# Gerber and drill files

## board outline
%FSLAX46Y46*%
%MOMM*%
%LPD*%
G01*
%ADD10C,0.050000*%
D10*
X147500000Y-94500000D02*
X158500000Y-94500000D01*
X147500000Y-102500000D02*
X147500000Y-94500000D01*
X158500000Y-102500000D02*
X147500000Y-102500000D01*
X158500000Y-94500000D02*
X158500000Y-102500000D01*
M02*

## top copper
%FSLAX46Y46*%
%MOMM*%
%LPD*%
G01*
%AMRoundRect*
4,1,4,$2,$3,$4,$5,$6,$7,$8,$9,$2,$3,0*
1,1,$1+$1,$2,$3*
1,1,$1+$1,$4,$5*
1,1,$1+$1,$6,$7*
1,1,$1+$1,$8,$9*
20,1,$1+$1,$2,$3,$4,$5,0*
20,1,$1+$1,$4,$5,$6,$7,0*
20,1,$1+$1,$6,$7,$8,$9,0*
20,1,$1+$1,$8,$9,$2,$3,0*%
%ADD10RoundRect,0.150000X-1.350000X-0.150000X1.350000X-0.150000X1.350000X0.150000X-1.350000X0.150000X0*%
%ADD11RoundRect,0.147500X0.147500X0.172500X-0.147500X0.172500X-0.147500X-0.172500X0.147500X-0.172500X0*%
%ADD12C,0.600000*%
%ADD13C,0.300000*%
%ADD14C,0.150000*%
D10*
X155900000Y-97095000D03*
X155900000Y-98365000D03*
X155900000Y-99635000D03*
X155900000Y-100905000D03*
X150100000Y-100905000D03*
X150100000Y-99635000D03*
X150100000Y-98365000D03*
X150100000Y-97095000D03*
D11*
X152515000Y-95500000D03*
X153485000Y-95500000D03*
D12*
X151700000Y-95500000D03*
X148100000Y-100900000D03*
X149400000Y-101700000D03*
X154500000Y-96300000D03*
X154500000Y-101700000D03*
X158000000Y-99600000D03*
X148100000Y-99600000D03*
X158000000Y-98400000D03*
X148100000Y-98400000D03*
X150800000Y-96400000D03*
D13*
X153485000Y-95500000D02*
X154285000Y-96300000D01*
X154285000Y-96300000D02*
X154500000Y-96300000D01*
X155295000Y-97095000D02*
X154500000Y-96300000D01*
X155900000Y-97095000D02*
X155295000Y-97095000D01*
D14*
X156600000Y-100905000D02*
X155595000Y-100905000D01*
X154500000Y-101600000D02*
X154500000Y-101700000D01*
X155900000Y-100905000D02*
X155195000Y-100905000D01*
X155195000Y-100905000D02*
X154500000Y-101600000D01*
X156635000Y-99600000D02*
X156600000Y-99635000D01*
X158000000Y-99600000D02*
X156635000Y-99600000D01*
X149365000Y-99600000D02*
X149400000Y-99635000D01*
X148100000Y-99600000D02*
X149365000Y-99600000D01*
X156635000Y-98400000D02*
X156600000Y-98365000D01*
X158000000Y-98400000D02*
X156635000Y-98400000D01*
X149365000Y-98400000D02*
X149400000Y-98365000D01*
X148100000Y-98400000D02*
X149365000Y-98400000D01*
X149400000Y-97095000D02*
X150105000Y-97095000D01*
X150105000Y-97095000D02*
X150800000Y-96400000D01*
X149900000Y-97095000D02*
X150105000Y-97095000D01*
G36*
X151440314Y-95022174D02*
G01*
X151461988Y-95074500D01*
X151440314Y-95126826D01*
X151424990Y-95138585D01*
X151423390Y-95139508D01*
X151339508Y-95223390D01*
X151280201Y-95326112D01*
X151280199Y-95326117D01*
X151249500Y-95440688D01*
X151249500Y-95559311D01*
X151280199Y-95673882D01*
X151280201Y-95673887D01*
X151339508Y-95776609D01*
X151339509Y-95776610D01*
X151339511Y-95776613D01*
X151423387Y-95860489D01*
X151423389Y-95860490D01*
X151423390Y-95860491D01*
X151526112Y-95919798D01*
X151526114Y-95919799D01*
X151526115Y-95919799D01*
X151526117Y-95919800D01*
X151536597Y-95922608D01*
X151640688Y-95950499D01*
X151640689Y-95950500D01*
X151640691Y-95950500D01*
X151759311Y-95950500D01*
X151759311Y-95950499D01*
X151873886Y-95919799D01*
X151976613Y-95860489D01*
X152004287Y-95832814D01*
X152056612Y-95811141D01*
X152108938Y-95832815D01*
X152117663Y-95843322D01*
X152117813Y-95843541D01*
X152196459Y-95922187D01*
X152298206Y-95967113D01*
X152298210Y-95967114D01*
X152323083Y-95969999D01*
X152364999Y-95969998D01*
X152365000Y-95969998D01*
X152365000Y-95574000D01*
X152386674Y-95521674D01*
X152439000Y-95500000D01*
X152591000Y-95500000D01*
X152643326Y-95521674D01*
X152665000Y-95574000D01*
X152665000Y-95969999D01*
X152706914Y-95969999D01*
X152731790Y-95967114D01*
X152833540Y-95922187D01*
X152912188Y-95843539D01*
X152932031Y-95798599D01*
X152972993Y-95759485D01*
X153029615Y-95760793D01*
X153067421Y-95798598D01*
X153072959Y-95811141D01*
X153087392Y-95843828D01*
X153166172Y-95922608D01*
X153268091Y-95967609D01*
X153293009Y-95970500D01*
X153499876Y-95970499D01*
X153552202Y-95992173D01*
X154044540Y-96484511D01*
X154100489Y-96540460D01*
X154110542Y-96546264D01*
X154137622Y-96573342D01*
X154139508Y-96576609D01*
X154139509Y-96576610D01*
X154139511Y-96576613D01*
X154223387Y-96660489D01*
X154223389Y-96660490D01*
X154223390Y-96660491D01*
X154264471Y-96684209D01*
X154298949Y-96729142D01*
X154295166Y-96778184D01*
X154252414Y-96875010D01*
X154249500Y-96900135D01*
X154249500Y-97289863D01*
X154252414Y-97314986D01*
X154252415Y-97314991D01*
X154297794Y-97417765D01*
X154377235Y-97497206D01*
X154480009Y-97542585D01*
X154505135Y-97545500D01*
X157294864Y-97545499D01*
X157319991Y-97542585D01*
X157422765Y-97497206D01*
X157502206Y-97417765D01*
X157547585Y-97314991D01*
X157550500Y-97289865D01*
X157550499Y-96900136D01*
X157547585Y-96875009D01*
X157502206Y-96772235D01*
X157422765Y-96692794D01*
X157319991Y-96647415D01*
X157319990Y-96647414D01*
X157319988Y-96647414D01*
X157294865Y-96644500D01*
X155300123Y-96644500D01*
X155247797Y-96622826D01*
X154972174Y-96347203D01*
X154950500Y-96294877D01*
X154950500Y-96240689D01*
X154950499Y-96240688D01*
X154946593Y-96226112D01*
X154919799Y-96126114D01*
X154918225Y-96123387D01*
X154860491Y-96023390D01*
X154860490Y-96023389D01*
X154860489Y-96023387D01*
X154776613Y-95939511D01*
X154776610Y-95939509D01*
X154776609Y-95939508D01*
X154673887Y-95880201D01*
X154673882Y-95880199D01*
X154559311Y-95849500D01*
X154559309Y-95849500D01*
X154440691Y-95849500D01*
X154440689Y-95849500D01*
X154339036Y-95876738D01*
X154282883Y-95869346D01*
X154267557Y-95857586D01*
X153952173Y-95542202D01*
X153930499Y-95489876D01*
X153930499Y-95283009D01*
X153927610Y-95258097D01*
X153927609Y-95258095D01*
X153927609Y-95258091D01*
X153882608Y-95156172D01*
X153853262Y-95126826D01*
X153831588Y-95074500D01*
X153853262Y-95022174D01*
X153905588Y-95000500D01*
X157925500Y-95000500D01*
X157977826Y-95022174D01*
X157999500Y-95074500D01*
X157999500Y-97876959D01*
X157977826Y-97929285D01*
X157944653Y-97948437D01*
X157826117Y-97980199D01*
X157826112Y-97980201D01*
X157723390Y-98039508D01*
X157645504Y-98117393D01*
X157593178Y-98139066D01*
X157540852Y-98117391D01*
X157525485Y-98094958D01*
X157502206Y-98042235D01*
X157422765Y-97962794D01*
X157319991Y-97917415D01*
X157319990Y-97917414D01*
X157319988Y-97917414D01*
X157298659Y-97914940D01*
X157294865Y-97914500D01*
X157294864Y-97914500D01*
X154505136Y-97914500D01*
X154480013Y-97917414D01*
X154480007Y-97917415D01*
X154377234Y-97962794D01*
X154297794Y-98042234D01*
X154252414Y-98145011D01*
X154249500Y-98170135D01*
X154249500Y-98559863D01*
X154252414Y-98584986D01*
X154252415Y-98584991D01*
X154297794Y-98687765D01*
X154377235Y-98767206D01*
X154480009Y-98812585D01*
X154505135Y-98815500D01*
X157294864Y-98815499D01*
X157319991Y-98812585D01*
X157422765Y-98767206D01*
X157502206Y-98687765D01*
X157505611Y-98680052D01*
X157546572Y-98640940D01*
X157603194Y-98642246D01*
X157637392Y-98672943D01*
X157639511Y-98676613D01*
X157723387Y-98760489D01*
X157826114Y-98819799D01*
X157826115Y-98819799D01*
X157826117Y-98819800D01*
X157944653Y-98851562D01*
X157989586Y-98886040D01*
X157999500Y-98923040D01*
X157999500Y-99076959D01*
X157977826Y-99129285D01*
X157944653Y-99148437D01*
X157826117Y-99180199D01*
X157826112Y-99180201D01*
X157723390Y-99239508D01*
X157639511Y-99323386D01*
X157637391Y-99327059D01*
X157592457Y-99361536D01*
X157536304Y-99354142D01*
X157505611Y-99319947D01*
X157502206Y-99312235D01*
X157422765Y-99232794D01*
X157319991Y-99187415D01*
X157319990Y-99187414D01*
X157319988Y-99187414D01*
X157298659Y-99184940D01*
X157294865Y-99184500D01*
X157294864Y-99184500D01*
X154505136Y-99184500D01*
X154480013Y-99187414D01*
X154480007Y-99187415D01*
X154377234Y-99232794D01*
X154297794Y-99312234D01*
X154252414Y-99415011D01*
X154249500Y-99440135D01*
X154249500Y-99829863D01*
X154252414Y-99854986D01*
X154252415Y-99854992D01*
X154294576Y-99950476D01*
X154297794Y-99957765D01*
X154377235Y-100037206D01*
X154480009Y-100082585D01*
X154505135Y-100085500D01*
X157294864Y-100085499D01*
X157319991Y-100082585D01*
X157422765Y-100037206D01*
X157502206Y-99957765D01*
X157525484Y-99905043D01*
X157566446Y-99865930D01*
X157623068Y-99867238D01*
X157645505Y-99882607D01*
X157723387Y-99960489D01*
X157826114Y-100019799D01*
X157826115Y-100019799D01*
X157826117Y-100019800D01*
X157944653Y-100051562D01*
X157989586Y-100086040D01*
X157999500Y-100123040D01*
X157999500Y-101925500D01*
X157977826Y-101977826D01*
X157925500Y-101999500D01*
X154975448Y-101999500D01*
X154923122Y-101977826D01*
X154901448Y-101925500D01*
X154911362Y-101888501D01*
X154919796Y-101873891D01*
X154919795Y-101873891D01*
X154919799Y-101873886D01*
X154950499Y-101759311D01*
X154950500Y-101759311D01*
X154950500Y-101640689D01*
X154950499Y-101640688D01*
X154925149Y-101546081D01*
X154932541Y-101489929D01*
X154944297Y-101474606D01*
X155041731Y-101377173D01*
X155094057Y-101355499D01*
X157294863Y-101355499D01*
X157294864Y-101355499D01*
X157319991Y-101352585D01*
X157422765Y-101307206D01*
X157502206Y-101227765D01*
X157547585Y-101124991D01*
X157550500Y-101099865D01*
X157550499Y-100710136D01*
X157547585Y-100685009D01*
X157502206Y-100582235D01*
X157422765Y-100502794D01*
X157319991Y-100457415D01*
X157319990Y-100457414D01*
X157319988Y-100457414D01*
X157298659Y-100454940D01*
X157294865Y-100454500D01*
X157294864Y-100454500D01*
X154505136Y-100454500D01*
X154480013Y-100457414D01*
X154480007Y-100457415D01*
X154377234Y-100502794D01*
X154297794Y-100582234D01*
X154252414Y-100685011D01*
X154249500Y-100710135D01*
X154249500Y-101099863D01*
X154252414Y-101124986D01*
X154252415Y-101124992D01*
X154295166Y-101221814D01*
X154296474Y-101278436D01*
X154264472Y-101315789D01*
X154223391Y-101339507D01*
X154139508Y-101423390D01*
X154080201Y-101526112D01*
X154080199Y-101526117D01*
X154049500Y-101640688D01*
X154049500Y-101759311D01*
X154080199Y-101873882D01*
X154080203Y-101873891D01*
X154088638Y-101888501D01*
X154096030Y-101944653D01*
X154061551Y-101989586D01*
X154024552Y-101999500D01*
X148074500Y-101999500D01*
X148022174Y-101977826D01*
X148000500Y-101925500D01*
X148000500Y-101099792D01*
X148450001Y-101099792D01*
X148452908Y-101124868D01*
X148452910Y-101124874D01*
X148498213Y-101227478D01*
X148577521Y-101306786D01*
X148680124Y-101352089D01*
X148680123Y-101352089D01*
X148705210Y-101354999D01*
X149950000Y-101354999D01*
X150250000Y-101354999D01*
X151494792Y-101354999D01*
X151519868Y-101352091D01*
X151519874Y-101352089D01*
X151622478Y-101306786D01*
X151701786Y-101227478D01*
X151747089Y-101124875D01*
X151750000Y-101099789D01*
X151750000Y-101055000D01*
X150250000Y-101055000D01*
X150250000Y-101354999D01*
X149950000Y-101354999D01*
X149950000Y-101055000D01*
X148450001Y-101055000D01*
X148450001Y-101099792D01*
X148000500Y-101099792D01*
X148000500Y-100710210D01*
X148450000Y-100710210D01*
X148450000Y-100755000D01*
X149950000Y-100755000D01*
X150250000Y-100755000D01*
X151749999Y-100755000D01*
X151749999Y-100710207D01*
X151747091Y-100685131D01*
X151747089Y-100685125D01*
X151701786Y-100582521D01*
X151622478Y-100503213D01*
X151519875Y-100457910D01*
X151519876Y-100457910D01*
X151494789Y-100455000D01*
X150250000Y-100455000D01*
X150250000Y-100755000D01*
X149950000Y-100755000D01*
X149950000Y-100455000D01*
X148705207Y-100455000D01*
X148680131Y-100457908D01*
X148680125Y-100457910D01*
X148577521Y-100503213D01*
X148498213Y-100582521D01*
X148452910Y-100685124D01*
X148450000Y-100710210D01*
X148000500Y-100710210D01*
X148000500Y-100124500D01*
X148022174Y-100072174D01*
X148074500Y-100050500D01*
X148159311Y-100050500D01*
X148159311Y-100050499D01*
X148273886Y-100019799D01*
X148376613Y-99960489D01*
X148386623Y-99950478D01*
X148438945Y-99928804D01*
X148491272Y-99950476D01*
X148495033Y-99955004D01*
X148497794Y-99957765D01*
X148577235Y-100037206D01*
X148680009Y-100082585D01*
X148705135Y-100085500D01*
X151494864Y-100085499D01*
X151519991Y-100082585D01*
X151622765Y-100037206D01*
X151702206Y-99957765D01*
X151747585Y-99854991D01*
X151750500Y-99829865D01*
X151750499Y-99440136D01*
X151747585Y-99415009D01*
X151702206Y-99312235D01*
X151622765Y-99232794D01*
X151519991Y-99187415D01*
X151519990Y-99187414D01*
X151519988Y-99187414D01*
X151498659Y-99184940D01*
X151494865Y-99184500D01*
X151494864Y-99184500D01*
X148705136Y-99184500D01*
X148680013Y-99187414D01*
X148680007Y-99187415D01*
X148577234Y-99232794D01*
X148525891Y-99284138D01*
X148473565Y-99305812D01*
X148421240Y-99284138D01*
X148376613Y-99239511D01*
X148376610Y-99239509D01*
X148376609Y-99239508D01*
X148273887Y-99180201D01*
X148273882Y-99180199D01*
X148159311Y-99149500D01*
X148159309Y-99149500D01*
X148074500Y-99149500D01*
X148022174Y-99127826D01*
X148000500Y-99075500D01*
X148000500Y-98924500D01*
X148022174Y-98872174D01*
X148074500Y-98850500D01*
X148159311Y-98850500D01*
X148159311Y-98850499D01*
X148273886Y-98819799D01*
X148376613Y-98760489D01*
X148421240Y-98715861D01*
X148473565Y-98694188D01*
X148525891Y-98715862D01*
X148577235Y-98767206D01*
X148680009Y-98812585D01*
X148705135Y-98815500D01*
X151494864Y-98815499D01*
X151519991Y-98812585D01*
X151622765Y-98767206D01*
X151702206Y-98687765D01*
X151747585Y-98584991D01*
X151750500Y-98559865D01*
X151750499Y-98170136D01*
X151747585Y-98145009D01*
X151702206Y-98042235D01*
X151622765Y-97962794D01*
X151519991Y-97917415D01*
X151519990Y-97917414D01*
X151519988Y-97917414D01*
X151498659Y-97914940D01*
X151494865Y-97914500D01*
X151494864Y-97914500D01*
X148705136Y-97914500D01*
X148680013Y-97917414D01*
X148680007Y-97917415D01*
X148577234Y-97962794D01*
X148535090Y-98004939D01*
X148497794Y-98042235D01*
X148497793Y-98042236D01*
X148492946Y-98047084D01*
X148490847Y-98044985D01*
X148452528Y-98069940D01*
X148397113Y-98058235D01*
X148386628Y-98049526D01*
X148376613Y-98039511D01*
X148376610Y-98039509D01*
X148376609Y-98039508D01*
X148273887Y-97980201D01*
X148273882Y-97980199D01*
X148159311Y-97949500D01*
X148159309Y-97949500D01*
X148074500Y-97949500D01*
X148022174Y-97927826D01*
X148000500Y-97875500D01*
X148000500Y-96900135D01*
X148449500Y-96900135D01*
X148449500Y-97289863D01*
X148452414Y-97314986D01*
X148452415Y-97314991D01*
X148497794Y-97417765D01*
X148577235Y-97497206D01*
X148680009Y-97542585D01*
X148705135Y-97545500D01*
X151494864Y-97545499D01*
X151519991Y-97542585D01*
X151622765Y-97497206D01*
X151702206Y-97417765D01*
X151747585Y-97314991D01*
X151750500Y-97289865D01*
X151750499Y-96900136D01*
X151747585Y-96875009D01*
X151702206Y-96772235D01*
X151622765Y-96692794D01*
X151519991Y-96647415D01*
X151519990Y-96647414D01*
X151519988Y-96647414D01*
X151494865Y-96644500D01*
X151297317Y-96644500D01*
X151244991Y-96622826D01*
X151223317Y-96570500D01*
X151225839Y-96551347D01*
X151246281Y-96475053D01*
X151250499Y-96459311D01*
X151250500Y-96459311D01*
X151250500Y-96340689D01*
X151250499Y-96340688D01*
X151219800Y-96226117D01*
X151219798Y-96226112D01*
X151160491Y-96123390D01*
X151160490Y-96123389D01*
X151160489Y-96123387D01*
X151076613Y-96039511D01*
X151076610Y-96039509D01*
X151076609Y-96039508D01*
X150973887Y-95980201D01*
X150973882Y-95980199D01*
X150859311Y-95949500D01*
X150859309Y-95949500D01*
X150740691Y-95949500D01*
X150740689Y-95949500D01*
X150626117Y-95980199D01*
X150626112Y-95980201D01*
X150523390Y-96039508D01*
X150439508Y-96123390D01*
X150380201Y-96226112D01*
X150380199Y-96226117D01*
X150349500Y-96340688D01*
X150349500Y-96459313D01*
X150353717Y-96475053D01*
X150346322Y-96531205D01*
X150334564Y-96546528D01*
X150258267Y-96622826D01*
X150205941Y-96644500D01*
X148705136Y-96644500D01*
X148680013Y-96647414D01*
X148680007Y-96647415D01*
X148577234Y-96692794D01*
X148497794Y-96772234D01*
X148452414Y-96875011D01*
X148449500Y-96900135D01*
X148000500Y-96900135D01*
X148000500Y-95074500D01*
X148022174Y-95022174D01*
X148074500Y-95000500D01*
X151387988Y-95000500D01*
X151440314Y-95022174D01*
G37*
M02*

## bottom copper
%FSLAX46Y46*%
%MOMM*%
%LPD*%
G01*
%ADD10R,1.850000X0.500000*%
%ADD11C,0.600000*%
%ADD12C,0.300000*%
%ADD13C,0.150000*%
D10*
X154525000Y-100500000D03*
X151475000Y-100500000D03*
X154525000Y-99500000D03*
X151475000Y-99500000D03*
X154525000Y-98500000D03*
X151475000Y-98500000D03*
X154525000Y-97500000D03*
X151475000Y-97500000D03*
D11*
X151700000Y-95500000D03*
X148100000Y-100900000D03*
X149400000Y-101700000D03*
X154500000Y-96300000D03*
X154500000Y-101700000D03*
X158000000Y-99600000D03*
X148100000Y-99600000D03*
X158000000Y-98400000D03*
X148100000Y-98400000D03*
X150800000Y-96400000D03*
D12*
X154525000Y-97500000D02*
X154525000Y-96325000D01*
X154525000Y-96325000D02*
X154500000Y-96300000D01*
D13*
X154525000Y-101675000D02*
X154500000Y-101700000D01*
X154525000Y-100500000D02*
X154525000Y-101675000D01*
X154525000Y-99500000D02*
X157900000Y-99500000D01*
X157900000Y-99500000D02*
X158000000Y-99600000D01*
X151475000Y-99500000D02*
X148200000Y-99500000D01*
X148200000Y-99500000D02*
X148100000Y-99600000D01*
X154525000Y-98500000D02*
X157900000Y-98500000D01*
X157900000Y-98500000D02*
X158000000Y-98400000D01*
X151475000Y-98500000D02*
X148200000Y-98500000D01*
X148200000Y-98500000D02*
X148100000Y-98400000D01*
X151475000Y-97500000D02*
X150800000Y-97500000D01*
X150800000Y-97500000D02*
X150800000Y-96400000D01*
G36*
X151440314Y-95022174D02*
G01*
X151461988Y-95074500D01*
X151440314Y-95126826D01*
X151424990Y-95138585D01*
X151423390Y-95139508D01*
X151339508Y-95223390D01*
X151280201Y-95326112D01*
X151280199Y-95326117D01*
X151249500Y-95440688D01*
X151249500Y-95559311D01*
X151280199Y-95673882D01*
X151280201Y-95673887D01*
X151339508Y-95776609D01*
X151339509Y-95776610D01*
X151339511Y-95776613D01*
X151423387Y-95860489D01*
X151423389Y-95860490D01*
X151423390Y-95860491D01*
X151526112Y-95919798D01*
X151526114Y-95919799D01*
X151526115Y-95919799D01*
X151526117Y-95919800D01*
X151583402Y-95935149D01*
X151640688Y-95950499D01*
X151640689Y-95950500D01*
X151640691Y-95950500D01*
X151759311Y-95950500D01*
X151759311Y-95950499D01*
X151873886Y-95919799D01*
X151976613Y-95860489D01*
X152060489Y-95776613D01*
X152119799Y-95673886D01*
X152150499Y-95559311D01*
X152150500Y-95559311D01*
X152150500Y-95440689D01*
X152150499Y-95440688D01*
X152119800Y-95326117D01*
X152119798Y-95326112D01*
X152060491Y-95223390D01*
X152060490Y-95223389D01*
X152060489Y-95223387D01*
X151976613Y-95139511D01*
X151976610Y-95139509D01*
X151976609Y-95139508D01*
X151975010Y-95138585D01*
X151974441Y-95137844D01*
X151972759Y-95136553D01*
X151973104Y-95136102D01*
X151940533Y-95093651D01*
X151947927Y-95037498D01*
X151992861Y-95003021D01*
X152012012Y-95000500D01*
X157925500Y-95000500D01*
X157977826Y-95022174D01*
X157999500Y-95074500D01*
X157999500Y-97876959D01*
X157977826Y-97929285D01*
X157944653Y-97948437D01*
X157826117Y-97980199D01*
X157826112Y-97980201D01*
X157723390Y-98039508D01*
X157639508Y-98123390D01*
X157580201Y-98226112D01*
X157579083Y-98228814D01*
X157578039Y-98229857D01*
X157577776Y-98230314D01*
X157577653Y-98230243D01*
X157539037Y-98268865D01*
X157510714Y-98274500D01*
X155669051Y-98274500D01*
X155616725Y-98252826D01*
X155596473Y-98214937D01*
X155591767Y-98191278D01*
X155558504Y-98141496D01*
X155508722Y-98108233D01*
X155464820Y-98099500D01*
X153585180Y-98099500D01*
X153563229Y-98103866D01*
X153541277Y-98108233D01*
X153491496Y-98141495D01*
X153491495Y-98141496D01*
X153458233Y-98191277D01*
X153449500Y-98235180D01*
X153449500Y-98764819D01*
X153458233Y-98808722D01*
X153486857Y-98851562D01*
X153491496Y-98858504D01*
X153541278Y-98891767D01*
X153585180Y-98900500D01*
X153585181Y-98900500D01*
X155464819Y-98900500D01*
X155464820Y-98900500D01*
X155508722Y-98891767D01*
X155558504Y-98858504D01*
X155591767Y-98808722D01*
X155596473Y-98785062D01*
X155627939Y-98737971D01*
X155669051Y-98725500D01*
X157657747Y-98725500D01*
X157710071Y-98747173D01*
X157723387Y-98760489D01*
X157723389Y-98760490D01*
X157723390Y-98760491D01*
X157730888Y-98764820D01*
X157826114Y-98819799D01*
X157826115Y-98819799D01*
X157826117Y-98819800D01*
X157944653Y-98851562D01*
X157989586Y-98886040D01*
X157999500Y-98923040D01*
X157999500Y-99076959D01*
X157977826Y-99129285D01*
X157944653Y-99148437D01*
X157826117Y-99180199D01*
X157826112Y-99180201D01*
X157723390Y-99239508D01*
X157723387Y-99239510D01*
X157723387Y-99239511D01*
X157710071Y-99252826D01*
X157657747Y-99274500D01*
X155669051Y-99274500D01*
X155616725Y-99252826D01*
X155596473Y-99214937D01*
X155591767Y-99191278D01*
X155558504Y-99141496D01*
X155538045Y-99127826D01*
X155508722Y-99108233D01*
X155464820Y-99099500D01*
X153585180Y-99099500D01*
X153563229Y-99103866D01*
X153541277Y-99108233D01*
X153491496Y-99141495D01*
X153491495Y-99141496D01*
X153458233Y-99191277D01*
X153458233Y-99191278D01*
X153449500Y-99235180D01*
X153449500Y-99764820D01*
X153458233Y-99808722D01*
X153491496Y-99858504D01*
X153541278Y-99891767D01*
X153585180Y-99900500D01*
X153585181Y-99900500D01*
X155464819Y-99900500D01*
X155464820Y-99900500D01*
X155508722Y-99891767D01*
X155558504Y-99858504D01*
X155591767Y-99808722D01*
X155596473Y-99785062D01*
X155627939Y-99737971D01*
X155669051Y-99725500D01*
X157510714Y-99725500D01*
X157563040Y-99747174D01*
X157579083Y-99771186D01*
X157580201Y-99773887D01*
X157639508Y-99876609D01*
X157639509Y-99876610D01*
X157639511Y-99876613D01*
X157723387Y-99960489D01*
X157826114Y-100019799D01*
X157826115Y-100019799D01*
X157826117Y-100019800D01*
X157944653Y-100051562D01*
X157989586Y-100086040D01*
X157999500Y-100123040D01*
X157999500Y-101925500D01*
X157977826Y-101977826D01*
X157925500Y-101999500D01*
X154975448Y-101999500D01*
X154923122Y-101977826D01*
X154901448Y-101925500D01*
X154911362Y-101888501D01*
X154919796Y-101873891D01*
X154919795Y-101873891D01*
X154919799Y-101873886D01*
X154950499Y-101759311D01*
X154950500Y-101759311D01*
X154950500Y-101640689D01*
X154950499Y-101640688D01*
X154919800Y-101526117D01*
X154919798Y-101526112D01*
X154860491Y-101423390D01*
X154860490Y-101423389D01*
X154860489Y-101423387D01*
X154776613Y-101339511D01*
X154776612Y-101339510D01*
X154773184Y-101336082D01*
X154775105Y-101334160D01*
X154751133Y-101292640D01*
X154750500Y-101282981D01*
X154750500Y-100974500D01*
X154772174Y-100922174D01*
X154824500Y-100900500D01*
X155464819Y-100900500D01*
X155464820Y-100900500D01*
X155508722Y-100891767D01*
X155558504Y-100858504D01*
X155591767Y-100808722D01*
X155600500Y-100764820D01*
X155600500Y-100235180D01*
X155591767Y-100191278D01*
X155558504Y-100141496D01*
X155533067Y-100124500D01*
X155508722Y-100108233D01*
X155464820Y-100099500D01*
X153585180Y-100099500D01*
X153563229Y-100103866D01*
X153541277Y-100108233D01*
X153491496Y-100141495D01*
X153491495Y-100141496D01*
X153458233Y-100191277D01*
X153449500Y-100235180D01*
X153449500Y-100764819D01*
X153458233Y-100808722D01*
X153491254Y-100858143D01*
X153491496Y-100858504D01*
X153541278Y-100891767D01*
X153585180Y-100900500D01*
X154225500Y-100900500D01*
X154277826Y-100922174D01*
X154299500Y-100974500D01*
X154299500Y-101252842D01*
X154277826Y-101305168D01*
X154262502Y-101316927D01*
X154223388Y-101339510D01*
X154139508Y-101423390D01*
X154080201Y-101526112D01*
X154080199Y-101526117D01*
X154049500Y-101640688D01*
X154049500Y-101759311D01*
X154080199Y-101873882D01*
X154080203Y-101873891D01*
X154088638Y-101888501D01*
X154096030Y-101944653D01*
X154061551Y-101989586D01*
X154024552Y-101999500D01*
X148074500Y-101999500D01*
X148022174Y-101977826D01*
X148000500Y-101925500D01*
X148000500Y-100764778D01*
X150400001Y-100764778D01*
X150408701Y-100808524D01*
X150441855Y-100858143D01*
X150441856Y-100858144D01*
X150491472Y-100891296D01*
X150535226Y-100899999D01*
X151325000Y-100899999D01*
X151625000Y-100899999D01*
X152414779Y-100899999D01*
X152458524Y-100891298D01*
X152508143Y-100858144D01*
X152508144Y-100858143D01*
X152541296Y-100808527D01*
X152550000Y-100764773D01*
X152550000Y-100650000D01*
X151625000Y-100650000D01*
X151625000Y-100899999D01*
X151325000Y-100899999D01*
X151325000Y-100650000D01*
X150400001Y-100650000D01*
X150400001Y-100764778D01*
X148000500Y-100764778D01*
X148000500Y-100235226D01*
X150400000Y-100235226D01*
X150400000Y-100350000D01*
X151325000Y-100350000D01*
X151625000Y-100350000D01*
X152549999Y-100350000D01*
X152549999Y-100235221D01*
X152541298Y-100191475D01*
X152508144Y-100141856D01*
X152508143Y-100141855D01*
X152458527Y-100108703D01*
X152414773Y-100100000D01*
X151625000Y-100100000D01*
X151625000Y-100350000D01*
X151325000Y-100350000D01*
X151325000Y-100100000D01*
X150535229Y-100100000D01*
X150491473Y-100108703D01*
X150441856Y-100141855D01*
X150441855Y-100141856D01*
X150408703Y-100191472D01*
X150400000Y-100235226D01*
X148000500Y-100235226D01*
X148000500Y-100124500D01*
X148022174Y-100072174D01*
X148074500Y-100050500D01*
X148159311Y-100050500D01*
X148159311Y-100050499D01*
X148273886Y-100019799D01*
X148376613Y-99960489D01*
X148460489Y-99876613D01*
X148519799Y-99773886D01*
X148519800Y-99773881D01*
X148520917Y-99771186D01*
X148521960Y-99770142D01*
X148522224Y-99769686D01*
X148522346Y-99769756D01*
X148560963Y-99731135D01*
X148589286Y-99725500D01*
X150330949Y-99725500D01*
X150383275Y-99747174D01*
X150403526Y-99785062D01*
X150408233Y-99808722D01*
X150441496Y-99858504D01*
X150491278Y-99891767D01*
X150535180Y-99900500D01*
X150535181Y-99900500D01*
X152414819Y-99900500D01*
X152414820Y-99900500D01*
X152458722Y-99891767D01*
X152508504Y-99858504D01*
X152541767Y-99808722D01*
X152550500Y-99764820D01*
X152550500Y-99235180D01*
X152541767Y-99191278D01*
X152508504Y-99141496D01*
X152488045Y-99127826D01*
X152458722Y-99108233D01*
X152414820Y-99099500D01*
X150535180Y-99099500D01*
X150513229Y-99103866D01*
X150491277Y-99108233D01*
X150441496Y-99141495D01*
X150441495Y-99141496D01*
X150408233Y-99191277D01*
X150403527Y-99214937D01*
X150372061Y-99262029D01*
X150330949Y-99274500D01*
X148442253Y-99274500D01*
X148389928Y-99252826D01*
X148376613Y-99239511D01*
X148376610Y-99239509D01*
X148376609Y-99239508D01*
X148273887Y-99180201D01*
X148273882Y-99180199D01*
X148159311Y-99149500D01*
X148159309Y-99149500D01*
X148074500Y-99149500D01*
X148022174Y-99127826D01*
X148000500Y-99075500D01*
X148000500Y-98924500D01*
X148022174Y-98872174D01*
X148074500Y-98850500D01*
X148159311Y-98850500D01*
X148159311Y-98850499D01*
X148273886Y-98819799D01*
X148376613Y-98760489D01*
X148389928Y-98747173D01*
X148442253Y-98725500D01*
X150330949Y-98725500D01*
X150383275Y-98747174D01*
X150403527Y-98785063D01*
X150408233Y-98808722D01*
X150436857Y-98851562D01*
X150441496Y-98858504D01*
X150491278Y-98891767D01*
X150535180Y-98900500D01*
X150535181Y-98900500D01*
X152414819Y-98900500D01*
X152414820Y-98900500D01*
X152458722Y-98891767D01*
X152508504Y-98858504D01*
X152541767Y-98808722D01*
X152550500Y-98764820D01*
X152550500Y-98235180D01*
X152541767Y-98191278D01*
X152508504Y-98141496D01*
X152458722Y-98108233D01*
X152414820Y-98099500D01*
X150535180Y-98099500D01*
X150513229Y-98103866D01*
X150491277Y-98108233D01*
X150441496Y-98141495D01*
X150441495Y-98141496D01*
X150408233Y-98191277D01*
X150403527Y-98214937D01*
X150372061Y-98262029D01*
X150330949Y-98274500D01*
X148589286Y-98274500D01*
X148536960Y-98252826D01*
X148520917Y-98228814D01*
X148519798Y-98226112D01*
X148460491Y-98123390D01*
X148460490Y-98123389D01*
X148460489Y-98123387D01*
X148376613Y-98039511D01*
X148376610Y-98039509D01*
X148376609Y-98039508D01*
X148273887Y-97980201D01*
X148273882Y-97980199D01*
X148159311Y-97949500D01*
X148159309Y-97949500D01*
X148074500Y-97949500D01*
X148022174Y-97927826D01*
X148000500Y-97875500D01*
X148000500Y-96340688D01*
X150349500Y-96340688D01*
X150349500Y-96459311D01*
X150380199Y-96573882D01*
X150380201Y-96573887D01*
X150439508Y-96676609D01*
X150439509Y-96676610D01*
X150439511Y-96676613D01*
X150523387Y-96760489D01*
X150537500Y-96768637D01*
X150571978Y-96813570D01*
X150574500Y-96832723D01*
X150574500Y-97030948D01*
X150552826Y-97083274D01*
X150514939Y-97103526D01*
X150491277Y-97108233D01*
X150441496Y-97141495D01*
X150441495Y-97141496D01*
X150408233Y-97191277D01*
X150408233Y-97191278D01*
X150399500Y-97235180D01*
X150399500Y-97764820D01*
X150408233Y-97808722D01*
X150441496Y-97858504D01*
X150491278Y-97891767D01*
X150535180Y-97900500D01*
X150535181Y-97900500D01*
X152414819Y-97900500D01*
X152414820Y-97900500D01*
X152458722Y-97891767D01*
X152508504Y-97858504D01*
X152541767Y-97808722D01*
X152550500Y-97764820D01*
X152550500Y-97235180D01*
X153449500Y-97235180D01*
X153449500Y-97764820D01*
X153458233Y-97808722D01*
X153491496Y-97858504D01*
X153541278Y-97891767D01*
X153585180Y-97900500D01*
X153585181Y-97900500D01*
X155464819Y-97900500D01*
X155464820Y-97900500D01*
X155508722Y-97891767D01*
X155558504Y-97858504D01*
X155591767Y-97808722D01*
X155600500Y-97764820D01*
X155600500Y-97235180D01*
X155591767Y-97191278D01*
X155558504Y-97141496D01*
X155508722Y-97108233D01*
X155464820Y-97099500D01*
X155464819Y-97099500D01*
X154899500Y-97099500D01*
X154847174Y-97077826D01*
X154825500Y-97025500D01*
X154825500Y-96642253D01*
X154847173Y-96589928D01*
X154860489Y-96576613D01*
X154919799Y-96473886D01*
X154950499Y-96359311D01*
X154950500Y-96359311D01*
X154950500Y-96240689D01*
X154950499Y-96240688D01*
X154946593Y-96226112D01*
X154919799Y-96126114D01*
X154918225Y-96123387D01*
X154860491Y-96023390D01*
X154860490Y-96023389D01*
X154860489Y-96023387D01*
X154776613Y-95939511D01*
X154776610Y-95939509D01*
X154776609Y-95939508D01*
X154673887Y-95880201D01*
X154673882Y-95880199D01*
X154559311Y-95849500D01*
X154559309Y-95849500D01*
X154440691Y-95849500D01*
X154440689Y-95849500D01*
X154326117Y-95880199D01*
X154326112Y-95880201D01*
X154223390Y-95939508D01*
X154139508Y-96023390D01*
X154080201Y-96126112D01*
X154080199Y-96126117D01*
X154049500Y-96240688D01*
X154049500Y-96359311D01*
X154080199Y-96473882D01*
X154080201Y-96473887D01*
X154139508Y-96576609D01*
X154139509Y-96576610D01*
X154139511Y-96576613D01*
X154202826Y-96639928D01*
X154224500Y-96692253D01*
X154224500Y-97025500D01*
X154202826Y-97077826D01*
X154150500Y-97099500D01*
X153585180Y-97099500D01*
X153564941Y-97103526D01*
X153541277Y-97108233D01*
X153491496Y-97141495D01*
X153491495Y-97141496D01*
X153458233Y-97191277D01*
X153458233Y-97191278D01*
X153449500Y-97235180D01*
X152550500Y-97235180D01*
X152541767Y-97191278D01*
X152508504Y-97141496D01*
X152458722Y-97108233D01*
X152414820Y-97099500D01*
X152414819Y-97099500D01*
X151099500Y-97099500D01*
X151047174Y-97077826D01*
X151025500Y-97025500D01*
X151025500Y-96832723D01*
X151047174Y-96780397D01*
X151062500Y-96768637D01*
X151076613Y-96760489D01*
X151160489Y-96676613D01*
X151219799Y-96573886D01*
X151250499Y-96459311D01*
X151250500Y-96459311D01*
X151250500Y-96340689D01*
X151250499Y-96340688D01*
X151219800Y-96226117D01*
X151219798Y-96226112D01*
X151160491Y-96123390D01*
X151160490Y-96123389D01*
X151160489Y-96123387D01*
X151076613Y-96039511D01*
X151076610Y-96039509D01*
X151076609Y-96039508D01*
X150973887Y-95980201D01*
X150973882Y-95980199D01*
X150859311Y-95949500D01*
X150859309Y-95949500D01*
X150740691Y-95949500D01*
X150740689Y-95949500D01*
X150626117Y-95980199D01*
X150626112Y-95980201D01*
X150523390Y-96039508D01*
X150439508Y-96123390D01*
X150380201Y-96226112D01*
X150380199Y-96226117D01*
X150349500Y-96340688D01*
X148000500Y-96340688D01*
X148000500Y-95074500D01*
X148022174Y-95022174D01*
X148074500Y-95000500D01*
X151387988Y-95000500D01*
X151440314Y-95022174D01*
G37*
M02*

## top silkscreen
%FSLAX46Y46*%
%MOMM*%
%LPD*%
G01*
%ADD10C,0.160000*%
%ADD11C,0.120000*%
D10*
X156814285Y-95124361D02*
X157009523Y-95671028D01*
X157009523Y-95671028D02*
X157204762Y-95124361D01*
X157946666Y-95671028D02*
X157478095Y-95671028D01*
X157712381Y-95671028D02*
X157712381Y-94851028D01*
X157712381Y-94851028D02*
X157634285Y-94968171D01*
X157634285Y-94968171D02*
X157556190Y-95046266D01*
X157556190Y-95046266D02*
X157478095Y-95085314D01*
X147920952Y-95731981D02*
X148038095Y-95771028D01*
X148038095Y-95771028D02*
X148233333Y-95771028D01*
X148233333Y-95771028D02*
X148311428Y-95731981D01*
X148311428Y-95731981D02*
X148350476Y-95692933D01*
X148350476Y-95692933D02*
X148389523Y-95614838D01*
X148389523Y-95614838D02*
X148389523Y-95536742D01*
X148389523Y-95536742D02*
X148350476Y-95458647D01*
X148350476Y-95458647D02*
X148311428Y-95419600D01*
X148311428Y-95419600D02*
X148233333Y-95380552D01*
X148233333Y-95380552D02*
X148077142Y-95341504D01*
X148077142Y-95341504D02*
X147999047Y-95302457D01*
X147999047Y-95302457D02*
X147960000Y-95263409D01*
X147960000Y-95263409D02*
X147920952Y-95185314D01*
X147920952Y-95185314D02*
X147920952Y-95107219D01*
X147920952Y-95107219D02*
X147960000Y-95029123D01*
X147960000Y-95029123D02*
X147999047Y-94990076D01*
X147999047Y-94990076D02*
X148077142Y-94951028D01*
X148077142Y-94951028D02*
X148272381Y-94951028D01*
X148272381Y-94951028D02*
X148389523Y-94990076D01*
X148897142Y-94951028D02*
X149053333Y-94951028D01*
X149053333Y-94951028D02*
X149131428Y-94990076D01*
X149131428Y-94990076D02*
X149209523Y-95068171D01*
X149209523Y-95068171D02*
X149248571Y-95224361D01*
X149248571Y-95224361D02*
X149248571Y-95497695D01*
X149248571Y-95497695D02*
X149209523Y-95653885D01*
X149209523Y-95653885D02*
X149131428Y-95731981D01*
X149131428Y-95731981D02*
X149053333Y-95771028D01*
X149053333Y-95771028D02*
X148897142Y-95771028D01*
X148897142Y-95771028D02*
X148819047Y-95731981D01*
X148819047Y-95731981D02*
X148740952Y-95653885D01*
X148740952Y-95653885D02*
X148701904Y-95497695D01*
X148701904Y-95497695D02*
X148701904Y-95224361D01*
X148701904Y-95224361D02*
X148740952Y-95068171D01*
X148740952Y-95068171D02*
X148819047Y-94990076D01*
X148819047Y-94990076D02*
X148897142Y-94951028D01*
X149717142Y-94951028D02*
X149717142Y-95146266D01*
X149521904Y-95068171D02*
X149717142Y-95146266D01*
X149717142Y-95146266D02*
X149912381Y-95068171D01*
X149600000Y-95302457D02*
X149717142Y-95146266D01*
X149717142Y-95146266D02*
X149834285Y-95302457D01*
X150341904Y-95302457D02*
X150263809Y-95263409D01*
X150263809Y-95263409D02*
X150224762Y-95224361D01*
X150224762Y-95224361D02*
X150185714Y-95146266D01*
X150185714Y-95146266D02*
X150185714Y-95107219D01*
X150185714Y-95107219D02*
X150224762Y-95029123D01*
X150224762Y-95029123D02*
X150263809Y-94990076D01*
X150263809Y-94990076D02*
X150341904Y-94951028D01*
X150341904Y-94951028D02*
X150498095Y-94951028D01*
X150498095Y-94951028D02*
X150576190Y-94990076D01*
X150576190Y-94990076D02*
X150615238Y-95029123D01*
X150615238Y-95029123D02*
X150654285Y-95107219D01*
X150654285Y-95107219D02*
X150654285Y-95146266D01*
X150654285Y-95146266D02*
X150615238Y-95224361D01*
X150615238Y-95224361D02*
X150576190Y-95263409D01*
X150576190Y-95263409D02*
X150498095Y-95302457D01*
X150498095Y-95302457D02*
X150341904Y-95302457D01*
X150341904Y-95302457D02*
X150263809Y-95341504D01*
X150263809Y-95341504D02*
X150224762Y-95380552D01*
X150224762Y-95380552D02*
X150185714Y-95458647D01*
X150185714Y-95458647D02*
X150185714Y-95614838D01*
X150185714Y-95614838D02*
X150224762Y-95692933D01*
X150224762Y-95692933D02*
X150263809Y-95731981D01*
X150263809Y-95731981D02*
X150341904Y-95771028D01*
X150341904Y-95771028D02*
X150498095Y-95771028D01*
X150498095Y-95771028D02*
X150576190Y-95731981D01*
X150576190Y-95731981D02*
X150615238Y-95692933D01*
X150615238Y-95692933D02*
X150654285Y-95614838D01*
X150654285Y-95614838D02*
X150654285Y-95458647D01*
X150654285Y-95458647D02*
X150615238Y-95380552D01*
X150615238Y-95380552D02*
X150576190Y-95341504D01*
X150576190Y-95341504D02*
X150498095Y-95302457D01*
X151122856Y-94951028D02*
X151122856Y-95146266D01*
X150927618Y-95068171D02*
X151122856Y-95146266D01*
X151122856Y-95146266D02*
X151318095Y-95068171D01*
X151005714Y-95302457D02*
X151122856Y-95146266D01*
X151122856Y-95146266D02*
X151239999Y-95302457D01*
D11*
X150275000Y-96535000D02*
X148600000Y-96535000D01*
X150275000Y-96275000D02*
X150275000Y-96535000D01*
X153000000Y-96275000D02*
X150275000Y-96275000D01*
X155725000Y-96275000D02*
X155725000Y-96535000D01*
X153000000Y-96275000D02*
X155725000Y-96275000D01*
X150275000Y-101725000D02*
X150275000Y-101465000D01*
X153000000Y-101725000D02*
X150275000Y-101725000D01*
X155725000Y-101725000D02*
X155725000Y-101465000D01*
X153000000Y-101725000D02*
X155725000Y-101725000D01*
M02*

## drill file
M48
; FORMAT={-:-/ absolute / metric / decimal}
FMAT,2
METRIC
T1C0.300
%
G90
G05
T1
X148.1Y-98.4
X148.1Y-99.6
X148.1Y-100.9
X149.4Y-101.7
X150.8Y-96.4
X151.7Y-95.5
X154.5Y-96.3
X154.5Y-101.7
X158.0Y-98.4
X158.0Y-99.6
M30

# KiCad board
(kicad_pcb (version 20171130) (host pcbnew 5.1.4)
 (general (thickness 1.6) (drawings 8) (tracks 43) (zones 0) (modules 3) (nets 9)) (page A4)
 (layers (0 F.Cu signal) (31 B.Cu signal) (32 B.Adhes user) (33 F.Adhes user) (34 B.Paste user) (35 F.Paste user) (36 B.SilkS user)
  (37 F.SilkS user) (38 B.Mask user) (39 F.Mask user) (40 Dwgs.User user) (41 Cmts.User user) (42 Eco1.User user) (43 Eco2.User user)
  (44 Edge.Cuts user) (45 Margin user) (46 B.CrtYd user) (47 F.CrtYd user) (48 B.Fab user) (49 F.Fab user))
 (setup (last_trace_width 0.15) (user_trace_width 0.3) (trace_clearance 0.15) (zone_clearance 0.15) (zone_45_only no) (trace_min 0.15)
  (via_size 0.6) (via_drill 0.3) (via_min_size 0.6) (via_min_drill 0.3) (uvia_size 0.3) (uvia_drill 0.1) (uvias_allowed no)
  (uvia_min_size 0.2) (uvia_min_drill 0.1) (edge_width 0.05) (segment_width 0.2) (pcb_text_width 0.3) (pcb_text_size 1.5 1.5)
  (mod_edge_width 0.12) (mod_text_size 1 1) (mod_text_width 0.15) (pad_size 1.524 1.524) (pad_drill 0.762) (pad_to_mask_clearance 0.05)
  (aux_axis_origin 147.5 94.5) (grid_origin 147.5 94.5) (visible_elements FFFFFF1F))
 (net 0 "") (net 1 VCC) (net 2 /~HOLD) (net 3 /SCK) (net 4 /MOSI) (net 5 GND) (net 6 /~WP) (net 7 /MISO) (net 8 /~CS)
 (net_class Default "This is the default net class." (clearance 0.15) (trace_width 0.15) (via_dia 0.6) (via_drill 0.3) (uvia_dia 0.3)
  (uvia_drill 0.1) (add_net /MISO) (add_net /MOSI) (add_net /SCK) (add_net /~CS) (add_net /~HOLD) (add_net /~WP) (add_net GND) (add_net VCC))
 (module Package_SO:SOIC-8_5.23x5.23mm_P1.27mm (layer F.Cu) (at 153 99)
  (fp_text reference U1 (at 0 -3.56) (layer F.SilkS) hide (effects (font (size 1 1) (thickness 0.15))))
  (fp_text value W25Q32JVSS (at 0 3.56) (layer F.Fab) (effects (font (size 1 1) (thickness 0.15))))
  (fp_line (start -2.725 -2.465) (end -4.4 -2.465) (layer F.SilkS) (width 0.12))
  (fp_line (start -2.725 -2.725) (end -2.725 -2.465) (layer F.SilkS) (width 0.12))
  (fp_line (start 0 -2.725) (end -2.725 -2.725) (layer F.SilkS) (width 0.12))
  (fp_line (start 2.725 -2.725) (end 2.725 -2.465) (layer F.SilkS) (width 0.12))
  (fp_line (start 0 -2.725) (end 2.725 -2.725) (layer F.SilkS) (width 0.12))
  (fp_line (start -2.725 2.725) (end -2.725 2.465) (layer F.SilkS) (width 0.12))
  (fp_line (start 0 2.725) (end -2.725 2.725) (layer F.SilkS) (width 0.12))
  (fp_line (start 2.725 2.725) (end 2.725 2.465) (layer F.SilkS) (width 0.12))
  (fp_line (start 0 2.725) (end 2.725 2.725) (layer F.SilkS) (width 0.12))
  (pad 8 smd roundrect (at 2.9 -1.905) (size 3 0.6) (layers F.Cu F.Paste F.Mask) (roundrect_rratio 0.25) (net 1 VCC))
  (pad 7 smd roundrect (at 2.9 -0.635) (size 3 0.6) (layers F.Cu F.Paste F.Mask) (roundrect_rratio 0.25) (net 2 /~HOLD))
  (pad 6 smd roundrect (at 2.9 0.635) (size 3 0.6) (layers F.Cu F.Paste F.Mask) (roundrect_rratio 0.25) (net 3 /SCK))
  (pad 5 smd roundrect (at 2.9 1.905) (size 3 0.6) (layers F.Cu F.Paste F.Mask) (roundrect_rratio 0.25) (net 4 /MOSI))
  (pad 4 smd roundrect (at -2.9 1.905) (size 3 0.6) (layers F.Cu F.Paste F.Mask) (roundrect_rratio 0.25) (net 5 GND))
  (pad 3 smd roundrect (at -2.9 0.635) (size 3 0.6) (layers F.Cu F.Paste F.Mask) (roundrect_rratio 0.25) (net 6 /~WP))
  (pad 2 smd roundrect (at -2.9 -0.635) (size 3 0.6) (layers F.Cu F.Paste F.Mask) (roundrect_rratio 0.25) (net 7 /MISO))
  (pad 1 smd roundrect (at -2.9 -1.905) (size 3 0.6) (layers F.Cu F.Paste F.Mask) (roundrect_rratio 0.25) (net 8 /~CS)))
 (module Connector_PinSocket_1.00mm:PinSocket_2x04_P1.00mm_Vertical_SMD (layer B.Cu) (at 153 99 180)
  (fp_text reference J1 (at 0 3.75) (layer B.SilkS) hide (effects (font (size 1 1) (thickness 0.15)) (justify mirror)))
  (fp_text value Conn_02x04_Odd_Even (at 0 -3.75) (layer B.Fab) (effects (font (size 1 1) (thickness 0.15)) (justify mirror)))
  (pad 8 smd rect (at -1.525 -1.5 180) (size 1.85 0.5) (layers B.Cu B.Paste B.Mask) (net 4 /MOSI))
  (pad 7 smd rect (at 1.525 -1.5 180) (size 1.85 0.5) (layers B.Cu B.Paste B.Mask) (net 5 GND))
  (pad 6 smd rect (at -1.525 -0.5 180) (size 1.85 0.5) (layers B.Cu B.Paste B.Mask) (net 3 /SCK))
  (pad 5 smd rect (at 1.525 -0.5 180) (size 1.85 0.5) (layers B.Cu B.Paste B.Mask) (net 6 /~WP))
  (pad 4 smd rect (at -1.525 0.5 180) (size 1.85 0.5) (layers B.Cu B.Paste B.Mask) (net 2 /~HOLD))
  (pad 3 smd rect (at 1.525 0.5 180) (size 1.85 0.5) (layers B.Cu B.Paste B.Mask) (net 7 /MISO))
  (pad 2 smd rect (at -1.525 1.5 180) (size 1.85 0.5) (layers B.Cu B.Paste B.Mask) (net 1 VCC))
  (pad 1 smd rect (at 1.525 1.5 180) (size 1.85 0.5) (layers B.Cu B.Paste B.Mask) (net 8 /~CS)))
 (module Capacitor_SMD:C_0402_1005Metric (layer F.Cu) (at 153 95.5 180)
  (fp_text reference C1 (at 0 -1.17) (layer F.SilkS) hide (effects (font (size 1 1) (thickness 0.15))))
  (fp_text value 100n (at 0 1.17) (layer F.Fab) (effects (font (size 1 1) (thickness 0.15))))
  (pad 2 smd roundrect (at 0.485 0 180) (size 0.59 0.64) (layers F.Cu F.Paste F.Mask) (roundrect_rratio 0.25) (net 5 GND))
  (pad 1 smd roundrect (at -0.485 0 180) (size 0.59 0.64) (layers F.Cu F.Paste F.Mask) (roundrect_rratio 0.25) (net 1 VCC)))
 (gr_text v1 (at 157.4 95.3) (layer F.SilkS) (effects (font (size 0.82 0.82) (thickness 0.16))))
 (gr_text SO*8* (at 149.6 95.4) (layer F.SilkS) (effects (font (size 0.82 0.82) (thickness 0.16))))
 (gr_line (start 147.5 94.5) (end 158.5 94.5) (layer Edge.Cuts) (width 0.05))
 (gr_line (start 147.5 102.5) (end 147.5 94.5) (layer Edge.Cuts) (width 0.05))
 (gr_line (start 158.5 102.5) (end 147.5 102.5) (layer Edge.Cuts) (width 0.05))
 (gr_line (start 158.5 94.5) (end 158.5 102.5) (layer Edge.Cuts) (width 0.05))
 (via (at 151.7 95.5) (size 0.6) (drill 0.3) (layers F.Cu B.Cu) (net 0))
 (via (at 148.1 100.9) (size 0.6) (drill 0.3) (layers F.Cu B.Cu) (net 5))
 (via (at 149.4 101.7) (size 0.6) (drill 0.3) (layers F.Cu B.Cu) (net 5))
 (segment (start 154.525 97.5) (end 154.525 96.325) (width 0.3) (layer B.Cu) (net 1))
 (segment (start 153.485 95.5) (end 154.285 96.3) (width 0.3) (layer F.Cu) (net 1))
 (segment (start 154.525 96.325) (end 154.5 96.3) (width 0.3) (layer B.Cu) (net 1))
 (segment (start 154.285 96.3) (end 154.5 96.3) (width 0.3) (layer F.Cu) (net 1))
 (via (at 154.5 96.3) (size 0.6) (drill 0.3) (layers F.Cu B.Cu) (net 1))
 (segment (start 155.295 97.095) (end 154.5 96.3) (width 0.3) (layer F.Cu) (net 1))
 (segment (start 155.9 97.095) (end 155.295 97.095) (width 0.3) (layer F.Cu) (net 1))
 (segment (start 156.6 100.905) (end 155.595 100.905) (width 0.15) (layer F.Cu) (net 4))
 (segment (start 154.525 101.675) (end 154.5 101.7) (width 0.15) (layer B.Cu) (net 4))
 (segment (start 154.525 100.5) (end 154.525 101.675) (width 0.15) (layer B.Cu) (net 4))
 (via (at 154.5 101.7) (size 0.6) (drill 0.3) (layers F.Cu B.Cu) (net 4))
 (segment (start 154.5 101.6) (end 154.5 101.7) (width 0.15) (layer F.Cu) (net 4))
 (segment (start 155.9 100.905) (end 155.195 100.905) (width 0.15) (layer F.Cu) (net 4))
 (segment (start 155.195 100.905) (end 154.5 101.6) (width 0.15) (layer F.Cu) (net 4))
 (via (at 158 99.6) (size 0.6) (drill 0.3) (layers F.Cu B.Cu) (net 3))
 (segment (start 154.525 99.5) (end 157.9 99.5) (width 0.15) (layer B.Cu) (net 3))
 (segment (start 157.9 99.5) (end 158 99.6) (width 0.15) (layer B.Cu) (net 3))
 (segment (start 156.635 99.6) (end 156.6 99.635) (width 0.15) (layer F.Cu) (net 3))
 (segment (start 158 99.6) (end 156.635 99.6) (width 0.15) (layer F.Cu) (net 3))
 (via (at 148.1 99.6) (size 0.6) (drill 0.3) (layers F.Cu B.Cu) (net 6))
 (segment (start 151.475 99.5) (end 148.2 99.5) (width 0.15) (layer B.Cu) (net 6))
 (segment (start 148.2 99.5) (end 148.1 99.6) (width 0.15) (layer B.Cu) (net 6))
 (segment (start 149.365 99.6) (end 149.4 99.635) (width 0.15) (layer F.Cu) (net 6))
 (segment (start 148.1 99.6) (end 149.365 99.6) (width 0.15) (layer F.Cu) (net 6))
 (via (at 158 98.4) (size 0.6) (drill 0.3) (layers F.Cu B.Cu) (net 2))
 (segment (start 154.525 98.5) (end 157.9 98.5) (width 0.15) (layer B.Cu) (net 2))
 (segment (start 157.9 98.5) (end 158 98.4) (width 0.15) (layer B.Cu) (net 2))
 (segment (start 156.635 98.4) (end 156.6 98.365) (width 0.15) (layer F.Cu) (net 2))
 (segment (start 158 98.4) (end 156.635 98.4) (width 0.15) (layer F.Cu) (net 2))
 (via (at 148.1 98.4) (size 0.6) (drill 0.3) (layers F.Cu B.Cu) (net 7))
 (segment (start 151.475 98.5) (end 148.2 98.5) (width 0.15) (layer B.Cu) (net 7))
 (segment (start 148.2 98.5) (end 148.1 98.4) (width 0.15) (layer B.Cu) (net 7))
 (segment (start 149.365 98.4) (end 149.4 98.365) (width 0.15) (layer F.Cu) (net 7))
 (segment (start 148.1 98.4) (end 149.365 98.4) (width 0.15) (layer F.Cu) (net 7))
 (segment (start 149.4 97.095) (end 150.105 97.095) (width 0.15) (layer F.Cu) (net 8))
 (segment (start 151.475 97.5) (end 150.8 97.5) (width 0.15) (layer B.Cu) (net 8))
 (segment (start 150.8 97.5) (end 150.8 96.4) (width 0.15) (layer B.Cu) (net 8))
 (via (at 150.8 96.4) (size 0.6) (drill 0.3) (layers F.Cu B.Cu) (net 8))
 (segment (start 150.105 97.095) (end 150.8 96.4) (width 0.15) (layer F.Cu) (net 8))
 (segment (start 149.9 97.095) (end 150.105 97.095) (width 0.15) (layer F.Cu) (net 8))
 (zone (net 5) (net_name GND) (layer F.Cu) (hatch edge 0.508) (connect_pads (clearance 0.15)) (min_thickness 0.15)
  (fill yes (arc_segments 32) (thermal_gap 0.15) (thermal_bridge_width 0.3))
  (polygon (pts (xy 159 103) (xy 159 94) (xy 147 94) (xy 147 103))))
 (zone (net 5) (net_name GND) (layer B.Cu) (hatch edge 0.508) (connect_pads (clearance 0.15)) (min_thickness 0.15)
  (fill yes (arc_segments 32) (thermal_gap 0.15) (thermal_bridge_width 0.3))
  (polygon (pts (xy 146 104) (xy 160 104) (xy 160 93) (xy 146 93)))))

